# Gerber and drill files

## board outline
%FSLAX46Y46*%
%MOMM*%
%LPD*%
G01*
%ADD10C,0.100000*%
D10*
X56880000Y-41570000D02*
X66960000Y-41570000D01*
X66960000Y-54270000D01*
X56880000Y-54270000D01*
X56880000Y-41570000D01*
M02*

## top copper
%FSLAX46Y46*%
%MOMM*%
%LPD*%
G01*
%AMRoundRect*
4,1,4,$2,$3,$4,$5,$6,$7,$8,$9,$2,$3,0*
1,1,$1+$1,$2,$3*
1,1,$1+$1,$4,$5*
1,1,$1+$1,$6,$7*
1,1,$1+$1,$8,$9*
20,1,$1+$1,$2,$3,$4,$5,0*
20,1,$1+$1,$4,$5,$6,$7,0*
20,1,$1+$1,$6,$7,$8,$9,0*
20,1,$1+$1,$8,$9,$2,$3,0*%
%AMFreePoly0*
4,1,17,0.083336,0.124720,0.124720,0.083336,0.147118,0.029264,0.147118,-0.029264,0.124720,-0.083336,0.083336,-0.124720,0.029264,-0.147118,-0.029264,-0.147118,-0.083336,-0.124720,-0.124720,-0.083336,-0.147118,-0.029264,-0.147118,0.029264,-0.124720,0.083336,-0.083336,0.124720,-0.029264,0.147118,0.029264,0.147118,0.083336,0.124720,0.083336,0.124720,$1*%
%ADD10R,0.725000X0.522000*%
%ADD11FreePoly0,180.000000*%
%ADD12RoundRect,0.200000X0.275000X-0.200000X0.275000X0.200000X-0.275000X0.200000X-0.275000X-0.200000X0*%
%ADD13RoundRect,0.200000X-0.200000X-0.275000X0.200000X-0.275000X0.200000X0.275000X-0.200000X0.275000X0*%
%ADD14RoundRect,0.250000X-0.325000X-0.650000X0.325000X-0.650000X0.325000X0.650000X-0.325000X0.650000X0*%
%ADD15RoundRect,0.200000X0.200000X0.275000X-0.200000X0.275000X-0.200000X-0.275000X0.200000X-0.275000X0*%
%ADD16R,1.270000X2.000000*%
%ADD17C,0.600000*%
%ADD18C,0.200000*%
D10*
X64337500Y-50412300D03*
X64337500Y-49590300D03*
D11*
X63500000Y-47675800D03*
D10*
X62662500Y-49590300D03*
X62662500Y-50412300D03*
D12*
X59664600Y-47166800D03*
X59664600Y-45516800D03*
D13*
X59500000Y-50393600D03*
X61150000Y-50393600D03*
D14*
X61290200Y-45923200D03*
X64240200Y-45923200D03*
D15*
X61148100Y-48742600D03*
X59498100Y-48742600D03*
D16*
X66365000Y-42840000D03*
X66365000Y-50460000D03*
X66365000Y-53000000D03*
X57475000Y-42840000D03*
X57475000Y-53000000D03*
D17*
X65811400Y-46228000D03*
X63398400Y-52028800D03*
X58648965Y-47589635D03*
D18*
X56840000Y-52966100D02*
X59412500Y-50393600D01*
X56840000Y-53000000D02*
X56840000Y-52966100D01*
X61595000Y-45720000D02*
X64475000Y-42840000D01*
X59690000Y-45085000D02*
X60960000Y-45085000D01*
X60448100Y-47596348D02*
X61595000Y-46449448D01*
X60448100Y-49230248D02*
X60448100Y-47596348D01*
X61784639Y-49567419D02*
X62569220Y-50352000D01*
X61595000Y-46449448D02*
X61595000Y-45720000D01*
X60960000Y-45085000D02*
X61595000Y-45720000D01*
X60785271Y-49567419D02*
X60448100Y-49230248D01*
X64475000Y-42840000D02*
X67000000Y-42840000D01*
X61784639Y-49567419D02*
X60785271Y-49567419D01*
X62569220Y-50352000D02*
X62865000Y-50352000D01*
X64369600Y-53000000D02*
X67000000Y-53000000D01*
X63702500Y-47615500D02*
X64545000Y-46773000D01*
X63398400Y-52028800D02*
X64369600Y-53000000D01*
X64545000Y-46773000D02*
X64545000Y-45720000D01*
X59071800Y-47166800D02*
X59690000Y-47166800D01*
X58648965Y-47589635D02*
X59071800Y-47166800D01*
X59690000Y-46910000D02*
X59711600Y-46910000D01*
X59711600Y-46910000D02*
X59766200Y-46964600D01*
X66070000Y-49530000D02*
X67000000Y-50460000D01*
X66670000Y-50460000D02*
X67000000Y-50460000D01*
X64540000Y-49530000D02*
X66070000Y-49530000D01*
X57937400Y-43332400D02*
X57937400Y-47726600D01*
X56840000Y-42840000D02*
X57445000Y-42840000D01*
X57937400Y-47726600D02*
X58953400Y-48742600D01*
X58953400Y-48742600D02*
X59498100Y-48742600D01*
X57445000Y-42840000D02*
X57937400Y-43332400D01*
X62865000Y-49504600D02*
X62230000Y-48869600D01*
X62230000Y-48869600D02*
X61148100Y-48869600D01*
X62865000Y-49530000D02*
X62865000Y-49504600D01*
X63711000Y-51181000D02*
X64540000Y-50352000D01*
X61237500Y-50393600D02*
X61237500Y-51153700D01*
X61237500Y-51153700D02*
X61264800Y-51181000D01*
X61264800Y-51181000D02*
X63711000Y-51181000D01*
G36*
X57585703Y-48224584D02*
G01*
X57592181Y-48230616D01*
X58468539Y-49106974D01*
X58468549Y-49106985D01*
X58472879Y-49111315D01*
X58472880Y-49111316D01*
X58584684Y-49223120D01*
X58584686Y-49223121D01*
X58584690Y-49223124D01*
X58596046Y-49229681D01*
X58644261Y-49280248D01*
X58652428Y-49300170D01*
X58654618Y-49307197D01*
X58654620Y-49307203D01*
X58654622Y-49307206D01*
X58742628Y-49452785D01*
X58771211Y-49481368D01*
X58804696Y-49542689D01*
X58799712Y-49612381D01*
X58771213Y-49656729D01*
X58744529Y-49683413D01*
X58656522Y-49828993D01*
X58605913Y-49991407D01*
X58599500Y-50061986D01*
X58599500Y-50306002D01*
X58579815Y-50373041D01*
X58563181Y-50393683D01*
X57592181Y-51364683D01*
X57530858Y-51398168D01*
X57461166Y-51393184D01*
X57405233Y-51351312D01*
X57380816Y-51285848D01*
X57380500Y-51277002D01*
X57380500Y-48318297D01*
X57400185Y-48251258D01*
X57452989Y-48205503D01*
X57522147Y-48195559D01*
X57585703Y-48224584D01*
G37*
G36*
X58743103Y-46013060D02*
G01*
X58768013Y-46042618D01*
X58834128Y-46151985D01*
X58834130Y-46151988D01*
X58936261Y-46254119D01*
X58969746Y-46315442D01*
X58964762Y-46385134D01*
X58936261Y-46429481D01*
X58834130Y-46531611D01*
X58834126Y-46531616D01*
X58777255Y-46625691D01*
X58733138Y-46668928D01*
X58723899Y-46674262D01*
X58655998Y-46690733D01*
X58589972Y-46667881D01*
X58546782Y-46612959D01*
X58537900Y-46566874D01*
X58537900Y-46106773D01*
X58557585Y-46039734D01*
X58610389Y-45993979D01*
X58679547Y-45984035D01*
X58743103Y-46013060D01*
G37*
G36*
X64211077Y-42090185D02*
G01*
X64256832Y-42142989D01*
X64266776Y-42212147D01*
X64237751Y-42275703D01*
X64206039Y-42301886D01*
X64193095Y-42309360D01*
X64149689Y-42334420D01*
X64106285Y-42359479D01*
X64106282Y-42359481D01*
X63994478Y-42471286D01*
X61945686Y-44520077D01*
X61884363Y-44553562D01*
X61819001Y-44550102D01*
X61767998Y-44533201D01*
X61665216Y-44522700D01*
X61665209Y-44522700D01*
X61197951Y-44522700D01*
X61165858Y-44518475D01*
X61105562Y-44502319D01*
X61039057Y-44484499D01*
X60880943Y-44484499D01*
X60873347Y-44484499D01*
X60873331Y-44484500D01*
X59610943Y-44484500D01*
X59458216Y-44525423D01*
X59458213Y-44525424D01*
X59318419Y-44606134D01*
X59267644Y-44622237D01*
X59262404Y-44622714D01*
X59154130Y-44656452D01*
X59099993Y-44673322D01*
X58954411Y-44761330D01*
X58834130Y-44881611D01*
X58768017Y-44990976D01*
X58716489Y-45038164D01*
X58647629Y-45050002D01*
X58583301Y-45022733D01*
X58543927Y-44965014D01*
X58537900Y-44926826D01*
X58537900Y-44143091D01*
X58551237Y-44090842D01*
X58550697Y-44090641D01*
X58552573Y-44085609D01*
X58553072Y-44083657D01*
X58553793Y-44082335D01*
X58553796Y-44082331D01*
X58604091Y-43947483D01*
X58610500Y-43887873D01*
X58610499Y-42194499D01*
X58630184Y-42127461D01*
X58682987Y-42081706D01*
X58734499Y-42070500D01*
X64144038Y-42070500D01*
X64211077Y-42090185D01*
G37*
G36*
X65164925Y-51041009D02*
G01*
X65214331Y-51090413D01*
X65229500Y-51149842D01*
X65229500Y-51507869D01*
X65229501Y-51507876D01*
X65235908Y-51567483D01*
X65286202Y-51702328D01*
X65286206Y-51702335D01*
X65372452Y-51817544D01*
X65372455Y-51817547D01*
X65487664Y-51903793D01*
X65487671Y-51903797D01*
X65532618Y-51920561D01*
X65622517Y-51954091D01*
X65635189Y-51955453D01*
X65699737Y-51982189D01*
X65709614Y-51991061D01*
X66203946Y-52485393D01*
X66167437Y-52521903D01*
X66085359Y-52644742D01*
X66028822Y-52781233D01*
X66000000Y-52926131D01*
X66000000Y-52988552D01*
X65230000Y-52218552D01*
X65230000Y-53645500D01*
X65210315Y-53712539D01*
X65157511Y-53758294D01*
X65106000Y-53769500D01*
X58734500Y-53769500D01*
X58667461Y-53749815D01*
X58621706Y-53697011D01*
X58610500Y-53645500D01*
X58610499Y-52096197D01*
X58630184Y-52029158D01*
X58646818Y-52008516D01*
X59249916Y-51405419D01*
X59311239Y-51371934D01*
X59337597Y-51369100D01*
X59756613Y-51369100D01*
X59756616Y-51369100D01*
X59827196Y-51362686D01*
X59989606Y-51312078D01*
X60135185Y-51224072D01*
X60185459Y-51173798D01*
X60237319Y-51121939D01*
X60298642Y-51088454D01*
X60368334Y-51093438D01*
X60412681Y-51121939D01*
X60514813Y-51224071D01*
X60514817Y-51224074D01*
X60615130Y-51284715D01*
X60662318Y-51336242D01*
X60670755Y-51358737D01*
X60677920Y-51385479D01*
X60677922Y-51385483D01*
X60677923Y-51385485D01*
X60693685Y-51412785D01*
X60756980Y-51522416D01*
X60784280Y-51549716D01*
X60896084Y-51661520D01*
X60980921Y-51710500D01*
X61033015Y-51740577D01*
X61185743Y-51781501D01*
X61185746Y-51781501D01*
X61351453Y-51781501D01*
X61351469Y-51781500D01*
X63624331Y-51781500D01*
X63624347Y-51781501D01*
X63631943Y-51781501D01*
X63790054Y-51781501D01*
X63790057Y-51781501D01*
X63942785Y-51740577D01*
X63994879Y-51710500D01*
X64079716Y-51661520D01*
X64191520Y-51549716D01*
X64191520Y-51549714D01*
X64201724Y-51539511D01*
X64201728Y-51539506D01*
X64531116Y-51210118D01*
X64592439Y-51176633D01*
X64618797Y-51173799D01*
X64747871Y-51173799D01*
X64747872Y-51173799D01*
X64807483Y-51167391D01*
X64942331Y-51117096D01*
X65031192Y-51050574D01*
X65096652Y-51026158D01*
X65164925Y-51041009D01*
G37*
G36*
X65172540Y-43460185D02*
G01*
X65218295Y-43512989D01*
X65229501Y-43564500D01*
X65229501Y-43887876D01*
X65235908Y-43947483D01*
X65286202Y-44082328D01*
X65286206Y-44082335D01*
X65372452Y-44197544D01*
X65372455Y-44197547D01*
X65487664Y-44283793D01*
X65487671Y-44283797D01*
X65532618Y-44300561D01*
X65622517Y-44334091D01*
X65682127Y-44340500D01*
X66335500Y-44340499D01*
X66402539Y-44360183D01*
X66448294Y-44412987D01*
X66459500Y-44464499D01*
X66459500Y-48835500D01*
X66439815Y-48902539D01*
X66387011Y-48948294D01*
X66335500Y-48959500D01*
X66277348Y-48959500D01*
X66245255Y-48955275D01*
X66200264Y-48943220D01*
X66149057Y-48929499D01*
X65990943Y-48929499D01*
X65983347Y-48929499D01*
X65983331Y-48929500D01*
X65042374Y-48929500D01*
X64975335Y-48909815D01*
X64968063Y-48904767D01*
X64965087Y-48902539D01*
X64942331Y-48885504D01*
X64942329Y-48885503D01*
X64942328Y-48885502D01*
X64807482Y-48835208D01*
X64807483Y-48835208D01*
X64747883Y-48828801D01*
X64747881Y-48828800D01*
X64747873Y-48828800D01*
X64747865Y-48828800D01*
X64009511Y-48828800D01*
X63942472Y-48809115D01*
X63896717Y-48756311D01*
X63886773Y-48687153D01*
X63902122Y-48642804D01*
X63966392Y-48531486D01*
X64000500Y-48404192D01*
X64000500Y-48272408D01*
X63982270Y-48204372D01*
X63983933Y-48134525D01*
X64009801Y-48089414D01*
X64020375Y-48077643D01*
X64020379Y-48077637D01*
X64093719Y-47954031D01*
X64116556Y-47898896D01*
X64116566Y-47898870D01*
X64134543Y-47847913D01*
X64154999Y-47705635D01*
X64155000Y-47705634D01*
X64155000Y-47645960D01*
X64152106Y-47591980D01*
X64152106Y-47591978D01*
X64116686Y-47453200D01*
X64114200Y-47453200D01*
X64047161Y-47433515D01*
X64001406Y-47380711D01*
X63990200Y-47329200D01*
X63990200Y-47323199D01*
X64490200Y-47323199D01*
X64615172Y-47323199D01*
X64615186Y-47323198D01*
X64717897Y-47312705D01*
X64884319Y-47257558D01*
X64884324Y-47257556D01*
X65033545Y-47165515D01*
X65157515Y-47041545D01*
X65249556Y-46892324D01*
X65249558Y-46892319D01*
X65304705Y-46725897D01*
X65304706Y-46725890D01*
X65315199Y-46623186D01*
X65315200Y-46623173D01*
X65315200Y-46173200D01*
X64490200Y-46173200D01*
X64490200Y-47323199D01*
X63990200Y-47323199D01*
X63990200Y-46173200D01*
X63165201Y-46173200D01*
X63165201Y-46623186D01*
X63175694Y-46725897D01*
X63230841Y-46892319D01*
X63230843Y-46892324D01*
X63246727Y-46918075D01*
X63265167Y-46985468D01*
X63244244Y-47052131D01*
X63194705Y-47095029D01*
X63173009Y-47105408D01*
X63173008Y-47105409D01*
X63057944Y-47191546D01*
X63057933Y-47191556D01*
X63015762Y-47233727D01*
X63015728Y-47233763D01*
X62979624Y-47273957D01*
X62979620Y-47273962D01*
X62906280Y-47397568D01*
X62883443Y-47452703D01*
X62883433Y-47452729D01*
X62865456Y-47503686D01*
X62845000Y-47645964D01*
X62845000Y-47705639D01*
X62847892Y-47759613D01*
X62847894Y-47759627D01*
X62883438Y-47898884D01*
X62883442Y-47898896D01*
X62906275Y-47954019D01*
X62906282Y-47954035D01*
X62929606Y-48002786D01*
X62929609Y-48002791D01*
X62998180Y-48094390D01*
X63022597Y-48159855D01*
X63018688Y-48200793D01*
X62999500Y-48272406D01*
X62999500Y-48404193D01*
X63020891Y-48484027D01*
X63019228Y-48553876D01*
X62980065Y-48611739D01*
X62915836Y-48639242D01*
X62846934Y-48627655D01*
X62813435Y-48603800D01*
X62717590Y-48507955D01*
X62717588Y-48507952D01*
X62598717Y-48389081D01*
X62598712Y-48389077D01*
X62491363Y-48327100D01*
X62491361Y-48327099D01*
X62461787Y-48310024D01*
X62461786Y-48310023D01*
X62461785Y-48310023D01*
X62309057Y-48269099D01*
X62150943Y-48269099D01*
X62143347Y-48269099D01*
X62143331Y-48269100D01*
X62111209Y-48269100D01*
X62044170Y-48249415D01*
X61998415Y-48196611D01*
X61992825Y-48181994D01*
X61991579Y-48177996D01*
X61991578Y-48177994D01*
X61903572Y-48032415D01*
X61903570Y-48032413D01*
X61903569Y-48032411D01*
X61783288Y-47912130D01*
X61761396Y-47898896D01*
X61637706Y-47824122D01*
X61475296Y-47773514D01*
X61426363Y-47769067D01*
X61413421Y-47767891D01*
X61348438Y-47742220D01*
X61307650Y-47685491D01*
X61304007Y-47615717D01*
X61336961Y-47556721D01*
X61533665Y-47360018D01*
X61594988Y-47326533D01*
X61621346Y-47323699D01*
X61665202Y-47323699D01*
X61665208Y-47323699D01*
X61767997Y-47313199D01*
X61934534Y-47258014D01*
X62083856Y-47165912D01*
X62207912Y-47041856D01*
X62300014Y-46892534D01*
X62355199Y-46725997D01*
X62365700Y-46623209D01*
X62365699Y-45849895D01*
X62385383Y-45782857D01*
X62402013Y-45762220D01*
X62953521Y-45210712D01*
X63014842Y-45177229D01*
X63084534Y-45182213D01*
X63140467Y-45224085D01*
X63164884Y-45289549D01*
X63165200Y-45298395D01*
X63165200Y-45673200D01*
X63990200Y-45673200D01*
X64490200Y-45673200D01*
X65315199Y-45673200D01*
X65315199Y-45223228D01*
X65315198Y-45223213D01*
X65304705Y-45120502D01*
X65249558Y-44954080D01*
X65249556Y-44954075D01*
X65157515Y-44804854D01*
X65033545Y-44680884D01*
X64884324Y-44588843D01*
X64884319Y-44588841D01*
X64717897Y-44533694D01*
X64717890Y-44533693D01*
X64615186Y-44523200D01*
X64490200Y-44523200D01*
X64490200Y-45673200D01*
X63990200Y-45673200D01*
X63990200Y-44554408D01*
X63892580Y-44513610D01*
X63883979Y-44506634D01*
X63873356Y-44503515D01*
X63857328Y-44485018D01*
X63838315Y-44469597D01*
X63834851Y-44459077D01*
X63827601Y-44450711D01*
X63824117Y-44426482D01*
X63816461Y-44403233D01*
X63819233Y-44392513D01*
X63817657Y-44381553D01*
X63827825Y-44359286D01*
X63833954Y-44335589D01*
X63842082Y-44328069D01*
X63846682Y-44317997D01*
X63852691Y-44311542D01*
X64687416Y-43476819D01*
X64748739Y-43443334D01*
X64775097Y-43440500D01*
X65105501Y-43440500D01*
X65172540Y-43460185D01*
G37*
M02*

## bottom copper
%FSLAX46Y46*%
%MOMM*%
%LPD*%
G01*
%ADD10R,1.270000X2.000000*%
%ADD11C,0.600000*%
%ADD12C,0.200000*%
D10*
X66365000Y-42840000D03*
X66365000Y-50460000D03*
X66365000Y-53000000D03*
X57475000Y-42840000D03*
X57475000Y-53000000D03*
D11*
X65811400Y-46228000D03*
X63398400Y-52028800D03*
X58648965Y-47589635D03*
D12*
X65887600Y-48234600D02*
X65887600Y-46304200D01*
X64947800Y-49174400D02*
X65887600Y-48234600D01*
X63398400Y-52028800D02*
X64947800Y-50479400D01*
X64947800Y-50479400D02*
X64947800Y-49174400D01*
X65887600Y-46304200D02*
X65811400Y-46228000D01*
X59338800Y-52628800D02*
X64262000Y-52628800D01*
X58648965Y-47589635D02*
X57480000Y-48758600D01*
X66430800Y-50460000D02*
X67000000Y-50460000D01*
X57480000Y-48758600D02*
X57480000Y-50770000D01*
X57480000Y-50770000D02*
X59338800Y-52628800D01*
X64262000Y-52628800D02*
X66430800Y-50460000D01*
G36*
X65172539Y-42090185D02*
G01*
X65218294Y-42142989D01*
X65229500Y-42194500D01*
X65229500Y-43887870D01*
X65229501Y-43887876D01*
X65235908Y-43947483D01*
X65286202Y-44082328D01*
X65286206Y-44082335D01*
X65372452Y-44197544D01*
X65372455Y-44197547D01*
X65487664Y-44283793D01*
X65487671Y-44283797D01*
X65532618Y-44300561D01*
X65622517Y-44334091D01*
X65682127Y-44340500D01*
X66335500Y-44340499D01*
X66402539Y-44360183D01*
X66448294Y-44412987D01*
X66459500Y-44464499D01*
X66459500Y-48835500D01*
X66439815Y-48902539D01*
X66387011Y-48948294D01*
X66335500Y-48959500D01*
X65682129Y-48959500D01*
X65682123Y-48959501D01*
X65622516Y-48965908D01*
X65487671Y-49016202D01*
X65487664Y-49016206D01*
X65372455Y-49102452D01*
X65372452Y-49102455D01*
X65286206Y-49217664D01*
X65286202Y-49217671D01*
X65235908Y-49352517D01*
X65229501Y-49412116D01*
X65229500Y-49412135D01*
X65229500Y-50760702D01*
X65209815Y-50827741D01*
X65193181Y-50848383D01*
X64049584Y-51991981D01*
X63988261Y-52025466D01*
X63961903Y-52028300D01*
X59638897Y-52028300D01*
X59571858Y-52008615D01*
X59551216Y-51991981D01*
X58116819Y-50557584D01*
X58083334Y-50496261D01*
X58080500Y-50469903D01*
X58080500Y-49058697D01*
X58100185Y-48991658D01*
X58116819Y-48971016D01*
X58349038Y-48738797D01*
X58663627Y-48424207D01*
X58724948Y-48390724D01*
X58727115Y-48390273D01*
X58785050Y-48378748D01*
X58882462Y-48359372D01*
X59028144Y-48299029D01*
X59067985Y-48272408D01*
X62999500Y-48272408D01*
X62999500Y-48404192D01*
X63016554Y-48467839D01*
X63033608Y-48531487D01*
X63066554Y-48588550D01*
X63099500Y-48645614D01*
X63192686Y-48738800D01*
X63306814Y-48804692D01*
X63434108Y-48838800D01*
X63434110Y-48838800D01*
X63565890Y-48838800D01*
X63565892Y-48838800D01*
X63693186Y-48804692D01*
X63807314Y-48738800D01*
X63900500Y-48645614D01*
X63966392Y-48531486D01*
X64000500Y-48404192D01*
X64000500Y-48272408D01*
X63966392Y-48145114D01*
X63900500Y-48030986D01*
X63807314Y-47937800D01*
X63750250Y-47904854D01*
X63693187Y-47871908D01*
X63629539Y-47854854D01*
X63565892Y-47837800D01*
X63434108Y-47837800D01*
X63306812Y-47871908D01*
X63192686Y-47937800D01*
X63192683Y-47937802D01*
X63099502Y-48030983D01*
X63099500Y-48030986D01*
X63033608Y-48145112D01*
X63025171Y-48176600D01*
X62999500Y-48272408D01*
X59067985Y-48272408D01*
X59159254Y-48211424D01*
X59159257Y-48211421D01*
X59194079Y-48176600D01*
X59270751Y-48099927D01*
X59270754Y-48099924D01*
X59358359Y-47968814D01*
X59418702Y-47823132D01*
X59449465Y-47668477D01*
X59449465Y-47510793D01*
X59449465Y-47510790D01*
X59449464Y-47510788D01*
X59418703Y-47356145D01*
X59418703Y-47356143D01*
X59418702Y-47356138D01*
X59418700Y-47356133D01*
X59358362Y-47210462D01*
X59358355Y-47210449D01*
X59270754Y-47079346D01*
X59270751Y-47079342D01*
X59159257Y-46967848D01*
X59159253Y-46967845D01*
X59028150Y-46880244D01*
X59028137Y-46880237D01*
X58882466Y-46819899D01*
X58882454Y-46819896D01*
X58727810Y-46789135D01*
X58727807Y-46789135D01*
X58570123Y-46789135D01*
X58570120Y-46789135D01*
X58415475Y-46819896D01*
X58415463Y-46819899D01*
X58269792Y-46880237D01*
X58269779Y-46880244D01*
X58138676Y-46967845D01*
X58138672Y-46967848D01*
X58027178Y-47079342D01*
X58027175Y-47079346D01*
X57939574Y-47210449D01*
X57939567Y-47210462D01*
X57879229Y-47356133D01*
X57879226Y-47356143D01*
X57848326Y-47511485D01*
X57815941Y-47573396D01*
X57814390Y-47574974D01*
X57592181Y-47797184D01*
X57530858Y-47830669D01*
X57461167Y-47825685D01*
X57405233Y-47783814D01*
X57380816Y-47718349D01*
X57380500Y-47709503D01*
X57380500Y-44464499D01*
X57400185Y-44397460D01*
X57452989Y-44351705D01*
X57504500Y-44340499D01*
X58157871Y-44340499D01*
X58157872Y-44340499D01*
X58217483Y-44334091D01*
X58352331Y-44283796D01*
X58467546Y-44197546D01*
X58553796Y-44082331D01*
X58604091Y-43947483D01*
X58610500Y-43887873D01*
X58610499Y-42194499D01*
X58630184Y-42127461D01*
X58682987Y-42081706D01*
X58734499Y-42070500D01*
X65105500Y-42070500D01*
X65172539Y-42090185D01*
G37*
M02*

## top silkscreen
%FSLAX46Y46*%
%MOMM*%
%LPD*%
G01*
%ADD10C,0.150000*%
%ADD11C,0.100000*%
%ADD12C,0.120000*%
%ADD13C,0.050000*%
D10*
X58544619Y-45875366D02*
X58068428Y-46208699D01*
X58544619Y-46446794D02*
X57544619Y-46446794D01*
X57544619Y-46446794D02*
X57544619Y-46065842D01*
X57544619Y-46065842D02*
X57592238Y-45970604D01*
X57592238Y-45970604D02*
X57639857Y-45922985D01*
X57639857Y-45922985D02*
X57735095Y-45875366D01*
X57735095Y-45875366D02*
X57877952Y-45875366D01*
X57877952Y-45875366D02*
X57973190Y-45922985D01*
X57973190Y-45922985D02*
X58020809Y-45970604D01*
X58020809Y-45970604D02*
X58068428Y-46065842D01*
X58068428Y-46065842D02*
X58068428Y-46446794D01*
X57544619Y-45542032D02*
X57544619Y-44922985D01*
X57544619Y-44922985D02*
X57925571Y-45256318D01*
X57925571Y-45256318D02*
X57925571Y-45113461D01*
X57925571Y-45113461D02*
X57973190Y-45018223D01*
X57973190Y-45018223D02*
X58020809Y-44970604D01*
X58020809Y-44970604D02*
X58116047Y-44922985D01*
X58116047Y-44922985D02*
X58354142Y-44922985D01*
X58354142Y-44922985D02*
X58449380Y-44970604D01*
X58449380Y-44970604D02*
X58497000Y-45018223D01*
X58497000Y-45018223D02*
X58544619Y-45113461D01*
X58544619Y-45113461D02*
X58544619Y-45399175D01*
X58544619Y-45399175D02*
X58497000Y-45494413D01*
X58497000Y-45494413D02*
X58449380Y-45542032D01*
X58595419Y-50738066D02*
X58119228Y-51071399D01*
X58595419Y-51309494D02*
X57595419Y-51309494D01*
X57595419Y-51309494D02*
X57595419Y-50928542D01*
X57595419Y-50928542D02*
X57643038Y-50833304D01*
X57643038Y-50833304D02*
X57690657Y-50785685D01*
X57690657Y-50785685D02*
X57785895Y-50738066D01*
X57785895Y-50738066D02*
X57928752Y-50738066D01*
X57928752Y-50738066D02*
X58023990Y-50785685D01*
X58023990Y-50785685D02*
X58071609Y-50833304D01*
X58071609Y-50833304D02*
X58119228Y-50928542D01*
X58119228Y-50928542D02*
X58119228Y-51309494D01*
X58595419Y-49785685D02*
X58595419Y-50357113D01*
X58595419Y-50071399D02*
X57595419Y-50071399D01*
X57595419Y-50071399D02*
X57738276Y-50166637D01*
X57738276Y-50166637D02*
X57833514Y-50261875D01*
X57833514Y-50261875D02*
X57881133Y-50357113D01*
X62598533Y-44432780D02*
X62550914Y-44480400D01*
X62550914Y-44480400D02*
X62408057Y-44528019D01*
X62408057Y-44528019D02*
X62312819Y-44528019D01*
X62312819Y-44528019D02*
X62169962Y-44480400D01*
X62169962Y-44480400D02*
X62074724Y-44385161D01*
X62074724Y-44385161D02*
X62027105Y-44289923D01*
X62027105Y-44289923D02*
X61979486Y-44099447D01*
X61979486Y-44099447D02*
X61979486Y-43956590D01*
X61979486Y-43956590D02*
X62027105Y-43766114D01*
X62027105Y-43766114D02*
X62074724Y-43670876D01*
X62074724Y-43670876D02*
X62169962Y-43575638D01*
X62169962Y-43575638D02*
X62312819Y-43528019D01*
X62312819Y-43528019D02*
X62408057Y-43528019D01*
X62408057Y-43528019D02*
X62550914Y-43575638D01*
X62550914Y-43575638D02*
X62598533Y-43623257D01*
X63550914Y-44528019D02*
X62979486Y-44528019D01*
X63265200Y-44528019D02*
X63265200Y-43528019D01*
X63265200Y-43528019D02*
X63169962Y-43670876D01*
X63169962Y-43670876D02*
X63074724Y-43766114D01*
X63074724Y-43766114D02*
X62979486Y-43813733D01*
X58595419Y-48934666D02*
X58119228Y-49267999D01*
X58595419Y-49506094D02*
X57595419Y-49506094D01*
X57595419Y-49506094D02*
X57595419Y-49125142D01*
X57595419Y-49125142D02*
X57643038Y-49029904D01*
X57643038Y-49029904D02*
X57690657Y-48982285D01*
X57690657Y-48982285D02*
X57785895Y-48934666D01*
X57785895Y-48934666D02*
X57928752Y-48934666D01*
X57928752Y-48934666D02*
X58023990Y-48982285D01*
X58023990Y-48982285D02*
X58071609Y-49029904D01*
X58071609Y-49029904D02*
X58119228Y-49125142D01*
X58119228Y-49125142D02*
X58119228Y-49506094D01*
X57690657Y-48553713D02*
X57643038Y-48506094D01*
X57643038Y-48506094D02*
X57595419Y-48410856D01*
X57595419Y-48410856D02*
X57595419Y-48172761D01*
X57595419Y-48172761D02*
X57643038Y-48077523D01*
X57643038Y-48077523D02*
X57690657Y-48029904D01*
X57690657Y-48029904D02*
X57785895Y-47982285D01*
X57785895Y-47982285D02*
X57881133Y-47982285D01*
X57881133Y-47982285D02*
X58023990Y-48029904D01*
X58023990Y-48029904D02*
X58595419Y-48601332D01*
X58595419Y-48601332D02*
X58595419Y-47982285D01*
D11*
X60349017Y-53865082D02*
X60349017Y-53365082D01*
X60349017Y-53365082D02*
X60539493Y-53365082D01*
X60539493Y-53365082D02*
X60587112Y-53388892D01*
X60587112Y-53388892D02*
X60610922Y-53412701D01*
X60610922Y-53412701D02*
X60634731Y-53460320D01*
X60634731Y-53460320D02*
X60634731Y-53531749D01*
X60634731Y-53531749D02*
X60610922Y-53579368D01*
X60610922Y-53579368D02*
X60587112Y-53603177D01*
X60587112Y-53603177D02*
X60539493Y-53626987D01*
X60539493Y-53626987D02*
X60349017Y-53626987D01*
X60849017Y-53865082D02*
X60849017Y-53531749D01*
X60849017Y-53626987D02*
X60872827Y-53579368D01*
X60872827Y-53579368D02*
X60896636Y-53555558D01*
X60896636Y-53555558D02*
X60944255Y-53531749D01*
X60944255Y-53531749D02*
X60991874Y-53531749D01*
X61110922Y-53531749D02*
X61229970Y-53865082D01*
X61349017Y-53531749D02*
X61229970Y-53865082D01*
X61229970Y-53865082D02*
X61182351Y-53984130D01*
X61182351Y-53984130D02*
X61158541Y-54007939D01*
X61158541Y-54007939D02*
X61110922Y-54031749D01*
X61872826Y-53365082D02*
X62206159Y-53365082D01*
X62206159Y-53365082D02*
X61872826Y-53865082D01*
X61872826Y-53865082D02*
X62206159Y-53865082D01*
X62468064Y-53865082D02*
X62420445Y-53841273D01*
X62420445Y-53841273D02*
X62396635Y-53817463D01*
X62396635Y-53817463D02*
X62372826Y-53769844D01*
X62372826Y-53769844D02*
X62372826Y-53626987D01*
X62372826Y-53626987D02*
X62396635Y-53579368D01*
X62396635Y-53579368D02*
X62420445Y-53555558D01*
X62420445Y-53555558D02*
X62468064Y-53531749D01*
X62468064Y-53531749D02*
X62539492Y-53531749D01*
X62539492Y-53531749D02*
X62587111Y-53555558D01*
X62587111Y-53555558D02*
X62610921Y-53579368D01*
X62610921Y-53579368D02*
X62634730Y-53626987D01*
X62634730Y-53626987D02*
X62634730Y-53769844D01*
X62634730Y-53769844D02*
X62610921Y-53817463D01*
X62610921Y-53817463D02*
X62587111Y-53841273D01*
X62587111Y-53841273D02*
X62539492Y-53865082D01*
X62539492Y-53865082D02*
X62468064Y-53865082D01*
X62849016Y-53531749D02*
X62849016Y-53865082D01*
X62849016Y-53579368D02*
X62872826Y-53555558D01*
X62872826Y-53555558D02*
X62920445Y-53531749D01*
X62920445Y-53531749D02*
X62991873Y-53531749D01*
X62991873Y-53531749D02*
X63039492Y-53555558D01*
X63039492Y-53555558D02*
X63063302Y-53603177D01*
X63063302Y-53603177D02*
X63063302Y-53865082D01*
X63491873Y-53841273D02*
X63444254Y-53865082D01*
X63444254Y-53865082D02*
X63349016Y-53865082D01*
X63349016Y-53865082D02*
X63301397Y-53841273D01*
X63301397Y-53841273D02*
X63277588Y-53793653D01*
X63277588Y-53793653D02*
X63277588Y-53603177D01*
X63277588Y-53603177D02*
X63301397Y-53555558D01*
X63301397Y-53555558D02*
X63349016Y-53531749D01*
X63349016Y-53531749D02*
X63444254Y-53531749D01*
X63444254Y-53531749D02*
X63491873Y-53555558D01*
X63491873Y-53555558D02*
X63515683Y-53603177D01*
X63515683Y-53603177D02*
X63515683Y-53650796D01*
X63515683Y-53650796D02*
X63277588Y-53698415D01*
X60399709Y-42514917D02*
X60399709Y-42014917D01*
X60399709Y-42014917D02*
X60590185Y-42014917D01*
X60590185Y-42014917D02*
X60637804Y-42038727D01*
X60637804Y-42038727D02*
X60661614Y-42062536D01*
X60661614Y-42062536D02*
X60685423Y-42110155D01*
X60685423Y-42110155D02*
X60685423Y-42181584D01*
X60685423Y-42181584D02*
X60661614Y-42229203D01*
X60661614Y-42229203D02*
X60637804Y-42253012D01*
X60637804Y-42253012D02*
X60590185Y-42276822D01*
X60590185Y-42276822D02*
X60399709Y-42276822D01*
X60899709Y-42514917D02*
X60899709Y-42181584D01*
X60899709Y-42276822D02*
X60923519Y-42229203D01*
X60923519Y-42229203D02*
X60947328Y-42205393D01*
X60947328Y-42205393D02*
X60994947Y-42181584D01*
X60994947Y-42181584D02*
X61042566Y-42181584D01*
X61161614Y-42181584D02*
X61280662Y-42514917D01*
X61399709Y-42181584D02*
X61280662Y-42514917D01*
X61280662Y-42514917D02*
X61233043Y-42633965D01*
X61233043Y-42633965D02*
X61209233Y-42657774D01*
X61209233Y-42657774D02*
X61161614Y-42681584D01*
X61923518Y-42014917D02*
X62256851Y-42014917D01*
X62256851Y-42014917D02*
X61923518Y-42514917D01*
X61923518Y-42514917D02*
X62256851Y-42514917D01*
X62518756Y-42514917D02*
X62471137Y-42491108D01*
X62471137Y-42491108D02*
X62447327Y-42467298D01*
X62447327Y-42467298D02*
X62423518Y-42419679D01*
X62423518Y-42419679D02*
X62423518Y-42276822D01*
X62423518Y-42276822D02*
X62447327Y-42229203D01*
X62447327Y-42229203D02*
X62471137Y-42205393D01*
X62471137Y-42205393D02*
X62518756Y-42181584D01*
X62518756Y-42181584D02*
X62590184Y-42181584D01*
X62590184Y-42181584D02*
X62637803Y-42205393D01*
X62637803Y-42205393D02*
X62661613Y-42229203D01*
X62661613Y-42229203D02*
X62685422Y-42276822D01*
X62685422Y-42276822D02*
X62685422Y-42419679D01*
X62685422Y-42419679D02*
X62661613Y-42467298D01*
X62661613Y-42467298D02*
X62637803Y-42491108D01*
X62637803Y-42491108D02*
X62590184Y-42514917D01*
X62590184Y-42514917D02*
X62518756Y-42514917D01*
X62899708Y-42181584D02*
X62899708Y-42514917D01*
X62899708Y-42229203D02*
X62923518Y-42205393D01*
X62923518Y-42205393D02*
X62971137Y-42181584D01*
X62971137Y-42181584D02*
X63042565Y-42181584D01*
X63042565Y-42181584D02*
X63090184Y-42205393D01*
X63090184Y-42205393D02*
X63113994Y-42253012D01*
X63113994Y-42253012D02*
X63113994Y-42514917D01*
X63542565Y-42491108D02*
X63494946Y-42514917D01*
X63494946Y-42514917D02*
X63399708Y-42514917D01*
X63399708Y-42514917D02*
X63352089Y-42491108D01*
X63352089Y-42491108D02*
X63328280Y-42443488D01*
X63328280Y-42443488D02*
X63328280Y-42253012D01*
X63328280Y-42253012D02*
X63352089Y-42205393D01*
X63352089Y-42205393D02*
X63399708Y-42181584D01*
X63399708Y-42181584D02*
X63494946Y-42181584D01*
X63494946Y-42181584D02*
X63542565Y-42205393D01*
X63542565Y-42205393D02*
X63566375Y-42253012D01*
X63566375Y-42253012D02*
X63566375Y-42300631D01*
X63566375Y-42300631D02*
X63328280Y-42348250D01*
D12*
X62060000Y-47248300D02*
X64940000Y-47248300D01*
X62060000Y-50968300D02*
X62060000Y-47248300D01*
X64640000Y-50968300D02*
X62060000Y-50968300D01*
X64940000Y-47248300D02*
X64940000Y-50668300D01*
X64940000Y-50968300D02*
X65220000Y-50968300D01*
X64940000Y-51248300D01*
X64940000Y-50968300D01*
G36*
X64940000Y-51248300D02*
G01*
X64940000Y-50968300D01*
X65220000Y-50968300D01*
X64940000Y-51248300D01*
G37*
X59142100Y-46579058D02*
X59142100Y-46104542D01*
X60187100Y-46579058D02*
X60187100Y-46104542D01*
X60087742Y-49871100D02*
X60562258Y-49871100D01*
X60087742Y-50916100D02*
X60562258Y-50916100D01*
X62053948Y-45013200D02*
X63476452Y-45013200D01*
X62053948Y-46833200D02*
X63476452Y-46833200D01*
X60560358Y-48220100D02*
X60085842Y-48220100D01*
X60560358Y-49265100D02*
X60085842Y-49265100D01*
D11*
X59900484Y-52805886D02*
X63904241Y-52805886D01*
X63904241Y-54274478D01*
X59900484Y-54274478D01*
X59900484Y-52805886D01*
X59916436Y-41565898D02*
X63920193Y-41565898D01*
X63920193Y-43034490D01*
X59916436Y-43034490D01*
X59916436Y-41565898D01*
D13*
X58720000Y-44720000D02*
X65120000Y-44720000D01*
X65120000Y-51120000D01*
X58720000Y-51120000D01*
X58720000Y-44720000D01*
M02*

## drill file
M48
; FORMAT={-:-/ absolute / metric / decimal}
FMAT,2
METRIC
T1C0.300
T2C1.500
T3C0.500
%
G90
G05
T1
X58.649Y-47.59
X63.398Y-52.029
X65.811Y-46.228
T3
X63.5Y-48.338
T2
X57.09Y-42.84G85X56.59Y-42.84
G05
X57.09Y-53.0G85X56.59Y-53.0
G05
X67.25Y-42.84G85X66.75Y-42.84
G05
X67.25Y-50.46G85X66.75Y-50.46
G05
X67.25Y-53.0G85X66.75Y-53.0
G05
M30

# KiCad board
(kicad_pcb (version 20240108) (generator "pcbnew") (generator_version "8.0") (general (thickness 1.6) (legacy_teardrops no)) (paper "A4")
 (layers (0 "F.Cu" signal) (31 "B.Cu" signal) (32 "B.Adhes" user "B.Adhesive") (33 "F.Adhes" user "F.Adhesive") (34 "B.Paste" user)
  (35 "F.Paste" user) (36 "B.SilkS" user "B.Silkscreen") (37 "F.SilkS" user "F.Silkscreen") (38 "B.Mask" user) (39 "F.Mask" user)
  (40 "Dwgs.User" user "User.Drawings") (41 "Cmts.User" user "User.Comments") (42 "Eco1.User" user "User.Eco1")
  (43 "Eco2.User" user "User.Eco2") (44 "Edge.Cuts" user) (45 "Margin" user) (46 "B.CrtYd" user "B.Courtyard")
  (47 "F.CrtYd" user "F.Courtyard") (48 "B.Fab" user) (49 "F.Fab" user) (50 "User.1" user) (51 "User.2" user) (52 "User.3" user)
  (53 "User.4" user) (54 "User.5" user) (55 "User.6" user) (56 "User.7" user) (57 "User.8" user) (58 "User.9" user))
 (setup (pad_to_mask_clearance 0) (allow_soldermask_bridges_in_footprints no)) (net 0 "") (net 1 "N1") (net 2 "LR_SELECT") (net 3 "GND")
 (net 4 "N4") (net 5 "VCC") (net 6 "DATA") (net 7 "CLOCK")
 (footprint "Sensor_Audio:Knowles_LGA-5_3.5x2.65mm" (layer "F.Cu") (at 63.5 49.1083 180)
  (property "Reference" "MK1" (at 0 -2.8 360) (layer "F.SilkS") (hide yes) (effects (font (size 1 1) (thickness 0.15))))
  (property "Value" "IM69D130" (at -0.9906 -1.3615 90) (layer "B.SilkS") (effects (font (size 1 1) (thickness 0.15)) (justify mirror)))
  (fp_line (start 1.44 1.86) (end -1.44 1.86) (stroke (width 0.12) (type solid)) (layer "F.SilkS"))
  (fp_line (start 1.44 -1.86) (end 1.44 1.86) (stroke (width 0.12) (type solid)) (layer "F.SilkS"))
  (fp_line (start -1.14 -1.86) (end 1.44 -1.86) (stroke (width 0.12) (type solid)) (layer "F.SilkS"))
  (fp_line (start -1.44 1.86) (end -1.44 -1.56) (stroke (width 0.12) (type solid)) (layer "F.SilkS"))
  (fp_poly
   (pts (xy -1.44 -1.86) (xy -1.72 -1.86) (xy -1.44 -2.14) (xy -1.44 -1.86)) (stroke (width 0.12) (type solid)) (fill solid)
   (layer "F.SilkS"))
  (pad "" np_thru_hole circle (at 0 0.77 180) (size 0.5 0.5) (drill 0.5) (layers "*.Cu" "*.Mask"))
  (pad "1" smd rect (at -0.8375 -1.304 180) (size 0.725 0.522) (layers "F.Cu" "F.Paste" "F.Mask") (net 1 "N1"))
  (pad "2" smd rect (at -0.8375 -0.482 180) (size 0.725 0.522) (layers "F.Cu" "F.Paste" "F.Mask") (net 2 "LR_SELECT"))
  (pad "3" smd custom (at 0 1.4325 180) (size 0.3 0.3) (layers "F.Cu" "F.Mask") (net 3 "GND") (zone_connect 0)
   (options (clearance outline) (anchor circle)) (primitives))
  (pad "4" smd rect (at 0.8375 -0.482 180) (size 0.725 0.522) (layers "F.Cu" "F.Paste" "F.Mask") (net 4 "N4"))
  (pad "5" smd rect (at 0.8375 -1.304 180) (size 0.725 0.522) (layers "F.Cu" "F.Paste" "F.Mask") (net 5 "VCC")))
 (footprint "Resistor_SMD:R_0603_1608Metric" (layer "F.Cu") (at 59.6646 46.3418 90)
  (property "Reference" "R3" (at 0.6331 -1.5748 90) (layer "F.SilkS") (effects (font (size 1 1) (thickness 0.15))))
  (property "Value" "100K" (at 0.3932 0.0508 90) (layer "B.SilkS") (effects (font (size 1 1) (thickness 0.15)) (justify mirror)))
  (fp_line (start -0.237258 -0.5225) (end 0.237258 -0.5225) (stroke (width 0.12) (type solid)) (layer "F.SilkS"))
  (fp_line (start -0.237258 0.5225) (end 0.237258 0.5225) (stroke (width 0.12) (type solid)) (layer "F.SilkS"))
  (pad "1" smd roundrect (at -0.825 0 90) (size 0.8 0.95) (layers "F.Cu" "F.Paste" "F.Mask") (roundrect_rratio 0.25) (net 2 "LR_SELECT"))
  (pad "2" smd roundrect (at 0.825 0 90) (size 0.8 0.95) (layers "F.Cu" "F.Paste" "F.Mask") (roundrect_rratio 0.25) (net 5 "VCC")))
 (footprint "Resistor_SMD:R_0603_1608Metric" (layer "F.Cu") (at 60.325 50.3936)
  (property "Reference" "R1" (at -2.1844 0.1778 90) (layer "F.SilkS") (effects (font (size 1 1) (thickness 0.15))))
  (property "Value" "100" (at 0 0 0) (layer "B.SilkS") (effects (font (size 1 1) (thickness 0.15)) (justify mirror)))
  (fp_line (start -0.237258 -0.5225) (end 0.237258 -0.5225) (stroke (width 0.12) (type solid)) (layer "F.SilkS"))
  (fp_line (start -0.237258 0.5225) (end 0.237258 0.5225) (stroke (width 0.12) (type solid)) (layer "F.SilkS"))
  (pad "1" smd roundrect (at -0.825 0) (size 0.8 0.95) (layers "F.Cu" "F.Paste" "F.Mask") (roundrect_rratio 0.25) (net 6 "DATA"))
  (pad "2" smd roundrect (at 0.825 0) (size 0.8 0.95) (layers "F.Cu" "F.Paste" "F.Mask") (roundrect_rratio 0.25) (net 1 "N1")))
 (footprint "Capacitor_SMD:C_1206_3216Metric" (layer "F.Cu") (at 62.7652 45.9232)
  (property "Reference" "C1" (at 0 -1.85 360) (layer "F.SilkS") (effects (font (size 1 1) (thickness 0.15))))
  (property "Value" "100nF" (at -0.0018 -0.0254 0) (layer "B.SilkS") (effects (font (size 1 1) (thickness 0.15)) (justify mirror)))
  (fp_line (start -0.711252 -0.91) (end 0.711252 -0.91) (stroke (width 0.12) (type solid)) (layer "F.SilkS"))
  (fp_line (start -0.711252 0.91) (end 0.711252 0.91) (stroke (width 0.12) (type solid)) (layer "F.SilkS"))
  (pad "1" smd roundrect (at -1.475 0) (size 1.15 1.8) (layers "F.Cu" "F.Paste" "F.Mask") (roundrect_rratio 0.217391) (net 5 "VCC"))
  (pad "2" smd roundrect (at 1.475 0) (size 1.15 1.8) (layers "F.Cu" "F.Paste" "F.Mask") (roundrect_rratio 0.217391) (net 3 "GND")))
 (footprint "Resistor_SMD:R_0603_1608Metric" (layer "F.Cu") (at 60.3231 48.7426 180)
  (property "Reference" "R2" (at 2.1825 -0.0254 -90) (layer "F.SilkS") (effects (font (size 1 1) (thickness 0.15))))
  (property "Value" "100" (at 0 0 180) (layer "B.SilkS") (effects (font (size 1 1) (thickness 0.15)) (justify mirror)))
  (fp_line (start -0.237258 0.5225) (end 0.237258 0.5225) (stroke (width 0.12) (type solid)) (layer "F.SilkS"))
  (fp_line (start -0.237258 -0.5225) (end 0.237258 -0.5225) (stroke (width 0.12) (type solid)) (layer "F.SilkS"))
  (pad "1" smd roundrect (at -0.825 0 180) (size 0.8 0.95) (layers "F.Cu" "F.Paste" "F.Mask") (roundrect_rratio 0.25) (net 4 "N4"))
  (pad "2" smd roundrect (at 0.825 0 180) (size 0.8 0.95) (layers "F.Cu" "F.Paste" "F.Mask") (roundrect_rratio 0.25) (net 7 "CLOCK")))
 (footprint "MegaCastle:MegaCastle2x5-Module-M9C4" (layer "B.Cu") (at 61.92 47.92 180)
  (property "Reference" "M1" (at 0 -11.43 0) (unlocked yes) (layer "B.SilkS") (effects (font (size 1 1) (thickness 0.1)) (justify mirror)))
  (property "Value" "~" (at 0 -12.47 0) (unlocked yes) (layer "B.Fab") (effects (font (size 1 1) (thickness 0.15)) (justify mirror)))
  (fp_rect (start -1.984241 -4.885886) (end 2.019516 -6.354478) (stroke (width 0.1) (type default)) (fill none) (layer "F.SilkS"))
  (fp_rect (start -2.000193 6.354102) (end 2.003564 4.88551) (stroke (width 0.1) (type default)) (fill none) (layer "F.SilkS"))
  (fp_rect (start -3.2 -3.2) (end 3.2 3.2) (stroke (width 0.05) (type default)) (fill none) (layer "F.SilkS"))
  (fp_rect (start -5.04 6.35) (end 5.04 -6.35) (stroke (width 0.1) (type default)) (fill none) (layer "Edge.Cuts"))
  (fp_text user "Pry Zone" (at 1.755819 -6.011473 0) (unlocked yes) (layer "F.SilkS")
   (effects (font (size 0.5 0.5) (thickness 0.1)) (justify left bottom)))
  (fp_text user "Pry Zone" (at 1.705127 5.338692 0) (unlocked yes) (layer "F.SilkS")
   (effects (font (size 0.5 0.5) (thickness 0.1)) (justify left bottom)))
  (pad "1" thru_hole rect (at -5.08 5.08 180) (size 1.27 2) (drill oval 2 1.5 (offset 0.635 0)) (layers "*.Cu" "*.Mask")
   (remove_unused_layers no) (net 5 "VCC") (thermal_bridge_angle 45))
  (pad "4" thru_hole rect (at -5.08 -2.54 180) (size 1.27 2) (drill oval 2 1.5 (offset 0.635 0)) (layers "*.Cu" "*.Mask")
   (remove_unused_layers no) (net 2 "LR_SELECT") (thermal_bridge_angle 45))
  (pad "5" thru_hole rect (at -5.08 -5.08 180) (size 1.27 2) (drill oval 2 1.5 (offset 0.635 0)) (layers "*.Cu" "*.Mask")
   (remove_unused_layers no) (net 3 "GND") (thermal_bridge_angle 45))
  (pad "6" thru_hole rect (at 5.08 5.08 180) (size 1.27 2) (drill oval 2 1.5 (offset -0.635 0)) (layers "*.Cu" "*.Mask")
   (remove_unused_layers no) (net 7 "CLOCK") (thermal_bridge_angle 45))
  (pad "10" thru_hole rect (at 5.08 -5.08 180) (size 1.27 2) (drill oval 2 1.5 (offset -0.635 0)) (layers "*.Cu" "*.Mask")
   (remove_unused_layers no) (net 6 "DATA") (thermal_bridge_angle 45))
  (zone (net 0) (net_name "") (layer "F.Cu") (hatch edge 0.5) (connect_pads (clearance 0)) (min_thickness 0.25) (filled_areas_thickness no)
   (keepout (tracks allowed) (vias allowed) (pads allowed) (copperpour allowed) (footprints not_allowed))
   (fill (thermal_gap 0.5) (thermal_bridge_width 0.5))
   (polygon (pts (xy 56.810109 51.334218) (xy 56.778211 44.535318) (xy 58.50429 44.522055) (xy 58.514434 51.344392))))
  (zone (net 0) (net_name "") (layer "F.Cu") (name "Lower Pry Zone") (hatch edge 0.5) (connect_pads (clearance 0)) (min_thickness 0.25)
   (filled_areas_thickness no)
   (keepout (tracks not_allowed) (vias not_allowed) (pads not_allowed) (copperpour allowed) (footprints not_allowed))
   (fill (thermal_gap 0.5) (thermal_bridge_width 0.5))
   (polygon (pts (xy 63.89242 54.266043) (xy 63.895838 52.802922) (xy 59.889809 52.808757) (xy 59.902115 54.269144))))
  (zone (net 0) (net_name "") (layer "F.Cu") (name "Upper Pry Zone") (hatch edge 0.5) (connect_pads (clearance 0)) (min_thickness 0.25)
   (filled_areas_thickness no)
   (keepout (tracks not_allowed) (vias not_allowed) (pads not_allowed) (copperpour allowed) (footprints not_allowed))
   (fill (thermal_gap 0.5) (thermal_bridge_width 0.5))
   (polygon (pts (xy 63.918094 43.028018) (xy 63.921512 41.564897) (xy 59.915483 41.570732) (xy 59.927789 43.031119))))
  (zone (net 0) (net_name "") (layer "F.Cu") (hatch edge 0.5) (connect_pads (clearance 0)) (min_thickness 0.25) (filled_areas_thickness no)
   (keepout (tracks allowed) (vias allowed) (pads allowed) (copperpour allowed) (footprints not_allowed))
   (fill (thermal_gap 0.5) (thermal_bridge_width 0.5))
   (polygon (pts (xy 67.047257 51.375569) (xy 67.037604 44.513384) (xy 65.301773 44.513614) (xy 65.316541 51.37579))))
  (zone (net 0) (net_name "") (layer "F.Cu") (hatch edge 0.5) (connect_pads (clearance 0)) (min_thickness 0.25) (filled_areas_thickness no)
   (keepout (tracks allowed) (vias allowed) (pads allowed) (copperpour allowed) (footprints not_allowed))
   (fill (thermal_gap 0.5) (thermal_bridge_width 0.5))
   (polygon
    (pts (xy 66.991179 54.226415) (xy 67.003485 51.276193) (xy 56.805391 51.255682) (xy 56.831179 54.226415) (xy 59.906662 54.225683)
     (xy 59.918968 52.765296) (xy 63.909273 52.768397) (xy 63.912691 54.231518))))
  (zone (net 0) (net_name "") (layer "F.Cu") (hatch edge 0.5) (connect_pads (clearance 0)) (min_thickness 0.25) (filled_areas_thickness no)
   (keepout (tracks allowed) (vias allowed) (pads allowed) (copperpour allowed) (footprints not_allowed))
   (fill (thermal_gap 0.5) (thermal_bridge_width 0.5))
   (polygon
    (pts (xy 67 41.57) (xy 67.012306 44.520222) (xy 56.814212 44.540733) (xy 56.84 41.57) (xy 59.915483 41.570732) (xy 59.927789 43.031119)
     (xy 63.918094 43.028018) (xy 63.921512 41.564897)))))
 (segment (start 56.84 52.9661) (end 59.4125 50.3936) (width 0.2) (layer "F.Cu") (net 6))
 (segment (start 56.84 53) (end 56.84 52.9661) (width 0.2) (layer "F.Cu") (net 6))
 (segment (start 61.595 45.72) (end 64.475 42.84) (width 0.2) (layer "F.Cu") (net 5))
 (segment (start 59.69 45.085) (end 60.96 45.085) (width 0.2) (layer "F.Cu") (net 5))
 (segment (start 60.4481 47.596348) (end 61.595 46.449448) (width 0.2) (layer "F.Cu") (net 5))
 (segment (start 60.4481 49.230248) (end 60.4481 47.596348) (width 0.2) (layer "F.Cu") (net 5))
 (segment (start 61.784639 49.567419) (end 62.56922 50.352) (width 0.2) (layer "F.Cu") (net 5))
 (segment (start 61.595 46.449448) (end 61.595 45.72) (width 0.2) (layer "F.Cu") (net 5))
 (segment (start 60.96 45.085) (end 61.595 45.72) (width 0.2) (layer "F.Cu") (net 5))
 (segment (start 60.785271 49.567419) (end 60.4481 49.230248) (width 0.2) (layer "F.Cu") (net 5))
 (segment (start 64.475 42.84) (end 67 42.84) (width 0.2) (layer "F.Cu") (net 5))
 (segment (start 61.784639 49.567419) (end 60.785271 49.567419) (width 0.2) (layer "F.Cu") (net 5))
 (segment (start 62.56922 50.352) (end 62.865 50.352) (width 0.2) (layer "F.Cu") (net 5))
 (segment (start 64.3696 53) (end 67 53) (width 0.2) (layer "F.Cu") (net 3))
 (segment (start 63.7025 47.6155) (end 64.545 46.773) (width 0.2) (layer "F.Cu") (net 3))
 (segment (start 63.3984 52.0288) (end 64.3696 53) (width 0.2) (layer "F.Cu") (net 3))
 (segment (start 64.545 46.773) (end 64.545 45.72) (width 0.2) (layer "F.Cu") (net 3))
 (via (at 65.8114 46.228) (size 0.6) (drill 0.3) (layers "F.Cu" "B.Cu") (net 3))
 (via (at 63.3984 52.0288) (size 0.6) (drill 0.3) (layers "F.Cu" "B.Cu") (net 3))
 (segment (start 65.8876 48.2346) (end 65.8876 46.3042) (width 0.2) (layer "B.Cu") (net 3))
 (segment (start 64.9478 49.1744) (end 65.8876 48.2346) (width 0.2) (layer "B.Cu") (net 3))
 (segment (start 63.3984 52.0288) (end 64.9478 50.4794) (width 0.2) (layer "B.Cu") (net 3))
 (segment (start 64.9478 50.4794) (end 64.9478 49.1744) (width 0.2) (layer "B.Cu") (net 3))
 (segment (start 65.8876 46.3042) (end 65.8114 46.228) (width 0.2) (layer "B.Cu") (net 3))
 (segment (start 59.0718 47.1668) (end 59.69 47.1668) (width 0.2) (layer "F.Cu") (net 2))
 (segment (start 58.648965 47.589635) (end 59.0718 47.1668) (width 0.2) (layer "F.Cu") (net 2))
 (segment (start 59.69 46.91) (end 59.7116 46.91) (width 0.2) (layer "F.Cu") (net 2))
 (segment (start 59.7116 46.91) (end 59.7662 46.9646) (width 0.2) (layer "F.Cu") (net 2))
 (segment (start 66.07 49.53) (end 67 50.46) (width 0.2) (layer "F.Cu") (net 2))
 (segment (start 66.67 50.46) (end 67 50.46) (width 0.2) (layer "F.Cu") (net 2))
 (segment (start 64.54 49.53) (end 66.07 49.53) (width 0.2) (layer "F.Cu") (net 2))
 (via (at 58.648965 47.589635) (size 0.6) (drill 0.3) (layers "F.Cu" "B.Cu") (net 2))
 (segment (start 59.3388 52.6288) (end 64.262 52.6288) (width 0.2) (layer "B.Cu") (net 2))
 (segment (start 58.648965 47.589635) (end 57.48 48.7586) (width 0.2) (layer "B.Cu") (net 2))
 (segment (start 66.4308 50.46) (end 67 50.46) (width 0.2) (layer "B.Cu") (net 2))
 (segment (start 57.48 48.7586) (end 57.48 50.77) (width 0.2) (layer "B.Cu") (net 2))
 (segment (start 57.48 50.77) (end 59.3388 52.6288) (width 0.2) (layer "B.Cu") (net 2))
 (segment (start 64.262 52.6288) (end 66.4308 50.46) (width 0.2) (layer "B.Cu") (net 2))
 (segment (start 57.9374 43.3324) (end 57.9374 47.7266) (width 0.2) (layer "F.Cu") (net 7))
 (segment (start 56.84 42.84) (end 57.445 42.84) (width 0.2) (layer "F.Cu") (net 7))
 (segment (start 57.9374 47.7266) (end 58.9534 48.7426) (width 0.2) (layer "F.Cu") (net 7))
 (segment (start 58.9534 48.7426) (end 59.4981 48.7426) (width 0.2) (layer "F.Cu") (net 7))
 (segment (start 57.445 42.84) (end 57.9374 43.3324) (width 0.2) (layer "F.Cu") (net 7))
 (segment (start 62.865 49.5046) (end 62.23 48.8696) (width 0.2) (layer "F.Cu") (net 4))
 (segment (start 62.23 48.8696) (end 61.1481 48.8696) (width 0.2) (layer "F.Cu") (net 4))
 (segment (start 62.865 49.53) (end 62.865 49.5046) (width 0.2) (layer "F.Cu") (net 4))
 (segment (start 63.711 51.181) (end 64.54 50.352) (width 0.2) (layer "F.Cu") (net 1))
 (segment (start 61.2375 50.3936) (end 61.2375 51.1537) (width 0.2) (layer "F.Cu") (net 1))
 (segment (start 61.2375 51.1537) (end 61.2648 51.181) (width 0.2) (layer "F.Cu") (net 1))
 (segment (start 61.2648 51.181) (end 63.711 51.181) (width 0.2) (layer "F.Cu") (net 1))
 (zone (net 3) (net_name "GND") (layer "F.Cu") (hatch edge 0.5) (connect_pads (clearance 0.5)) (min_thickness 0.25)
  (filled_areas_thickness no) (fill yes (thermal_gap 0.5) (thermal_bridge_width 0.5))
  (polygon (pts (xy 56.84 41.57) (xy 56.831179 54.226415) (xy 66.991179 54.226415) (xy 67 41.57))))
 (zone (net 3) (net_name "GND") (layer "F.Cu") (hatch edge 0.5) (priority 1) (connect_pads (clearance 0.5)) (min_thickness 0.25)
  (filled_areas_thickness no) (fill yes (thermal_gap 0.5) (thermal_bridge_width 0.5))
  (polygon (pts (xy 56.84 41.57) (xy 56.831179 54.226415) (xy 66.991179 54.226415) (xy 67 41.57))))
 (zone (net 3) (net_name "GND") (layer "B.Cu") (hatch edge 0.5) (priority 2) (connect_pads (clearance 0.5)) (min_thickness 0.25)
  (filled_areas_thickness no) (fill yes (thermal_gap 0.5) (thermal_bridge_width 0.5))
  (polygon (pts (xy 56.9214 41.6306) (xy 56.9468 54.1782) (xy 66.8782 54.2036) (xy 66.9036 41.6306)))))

